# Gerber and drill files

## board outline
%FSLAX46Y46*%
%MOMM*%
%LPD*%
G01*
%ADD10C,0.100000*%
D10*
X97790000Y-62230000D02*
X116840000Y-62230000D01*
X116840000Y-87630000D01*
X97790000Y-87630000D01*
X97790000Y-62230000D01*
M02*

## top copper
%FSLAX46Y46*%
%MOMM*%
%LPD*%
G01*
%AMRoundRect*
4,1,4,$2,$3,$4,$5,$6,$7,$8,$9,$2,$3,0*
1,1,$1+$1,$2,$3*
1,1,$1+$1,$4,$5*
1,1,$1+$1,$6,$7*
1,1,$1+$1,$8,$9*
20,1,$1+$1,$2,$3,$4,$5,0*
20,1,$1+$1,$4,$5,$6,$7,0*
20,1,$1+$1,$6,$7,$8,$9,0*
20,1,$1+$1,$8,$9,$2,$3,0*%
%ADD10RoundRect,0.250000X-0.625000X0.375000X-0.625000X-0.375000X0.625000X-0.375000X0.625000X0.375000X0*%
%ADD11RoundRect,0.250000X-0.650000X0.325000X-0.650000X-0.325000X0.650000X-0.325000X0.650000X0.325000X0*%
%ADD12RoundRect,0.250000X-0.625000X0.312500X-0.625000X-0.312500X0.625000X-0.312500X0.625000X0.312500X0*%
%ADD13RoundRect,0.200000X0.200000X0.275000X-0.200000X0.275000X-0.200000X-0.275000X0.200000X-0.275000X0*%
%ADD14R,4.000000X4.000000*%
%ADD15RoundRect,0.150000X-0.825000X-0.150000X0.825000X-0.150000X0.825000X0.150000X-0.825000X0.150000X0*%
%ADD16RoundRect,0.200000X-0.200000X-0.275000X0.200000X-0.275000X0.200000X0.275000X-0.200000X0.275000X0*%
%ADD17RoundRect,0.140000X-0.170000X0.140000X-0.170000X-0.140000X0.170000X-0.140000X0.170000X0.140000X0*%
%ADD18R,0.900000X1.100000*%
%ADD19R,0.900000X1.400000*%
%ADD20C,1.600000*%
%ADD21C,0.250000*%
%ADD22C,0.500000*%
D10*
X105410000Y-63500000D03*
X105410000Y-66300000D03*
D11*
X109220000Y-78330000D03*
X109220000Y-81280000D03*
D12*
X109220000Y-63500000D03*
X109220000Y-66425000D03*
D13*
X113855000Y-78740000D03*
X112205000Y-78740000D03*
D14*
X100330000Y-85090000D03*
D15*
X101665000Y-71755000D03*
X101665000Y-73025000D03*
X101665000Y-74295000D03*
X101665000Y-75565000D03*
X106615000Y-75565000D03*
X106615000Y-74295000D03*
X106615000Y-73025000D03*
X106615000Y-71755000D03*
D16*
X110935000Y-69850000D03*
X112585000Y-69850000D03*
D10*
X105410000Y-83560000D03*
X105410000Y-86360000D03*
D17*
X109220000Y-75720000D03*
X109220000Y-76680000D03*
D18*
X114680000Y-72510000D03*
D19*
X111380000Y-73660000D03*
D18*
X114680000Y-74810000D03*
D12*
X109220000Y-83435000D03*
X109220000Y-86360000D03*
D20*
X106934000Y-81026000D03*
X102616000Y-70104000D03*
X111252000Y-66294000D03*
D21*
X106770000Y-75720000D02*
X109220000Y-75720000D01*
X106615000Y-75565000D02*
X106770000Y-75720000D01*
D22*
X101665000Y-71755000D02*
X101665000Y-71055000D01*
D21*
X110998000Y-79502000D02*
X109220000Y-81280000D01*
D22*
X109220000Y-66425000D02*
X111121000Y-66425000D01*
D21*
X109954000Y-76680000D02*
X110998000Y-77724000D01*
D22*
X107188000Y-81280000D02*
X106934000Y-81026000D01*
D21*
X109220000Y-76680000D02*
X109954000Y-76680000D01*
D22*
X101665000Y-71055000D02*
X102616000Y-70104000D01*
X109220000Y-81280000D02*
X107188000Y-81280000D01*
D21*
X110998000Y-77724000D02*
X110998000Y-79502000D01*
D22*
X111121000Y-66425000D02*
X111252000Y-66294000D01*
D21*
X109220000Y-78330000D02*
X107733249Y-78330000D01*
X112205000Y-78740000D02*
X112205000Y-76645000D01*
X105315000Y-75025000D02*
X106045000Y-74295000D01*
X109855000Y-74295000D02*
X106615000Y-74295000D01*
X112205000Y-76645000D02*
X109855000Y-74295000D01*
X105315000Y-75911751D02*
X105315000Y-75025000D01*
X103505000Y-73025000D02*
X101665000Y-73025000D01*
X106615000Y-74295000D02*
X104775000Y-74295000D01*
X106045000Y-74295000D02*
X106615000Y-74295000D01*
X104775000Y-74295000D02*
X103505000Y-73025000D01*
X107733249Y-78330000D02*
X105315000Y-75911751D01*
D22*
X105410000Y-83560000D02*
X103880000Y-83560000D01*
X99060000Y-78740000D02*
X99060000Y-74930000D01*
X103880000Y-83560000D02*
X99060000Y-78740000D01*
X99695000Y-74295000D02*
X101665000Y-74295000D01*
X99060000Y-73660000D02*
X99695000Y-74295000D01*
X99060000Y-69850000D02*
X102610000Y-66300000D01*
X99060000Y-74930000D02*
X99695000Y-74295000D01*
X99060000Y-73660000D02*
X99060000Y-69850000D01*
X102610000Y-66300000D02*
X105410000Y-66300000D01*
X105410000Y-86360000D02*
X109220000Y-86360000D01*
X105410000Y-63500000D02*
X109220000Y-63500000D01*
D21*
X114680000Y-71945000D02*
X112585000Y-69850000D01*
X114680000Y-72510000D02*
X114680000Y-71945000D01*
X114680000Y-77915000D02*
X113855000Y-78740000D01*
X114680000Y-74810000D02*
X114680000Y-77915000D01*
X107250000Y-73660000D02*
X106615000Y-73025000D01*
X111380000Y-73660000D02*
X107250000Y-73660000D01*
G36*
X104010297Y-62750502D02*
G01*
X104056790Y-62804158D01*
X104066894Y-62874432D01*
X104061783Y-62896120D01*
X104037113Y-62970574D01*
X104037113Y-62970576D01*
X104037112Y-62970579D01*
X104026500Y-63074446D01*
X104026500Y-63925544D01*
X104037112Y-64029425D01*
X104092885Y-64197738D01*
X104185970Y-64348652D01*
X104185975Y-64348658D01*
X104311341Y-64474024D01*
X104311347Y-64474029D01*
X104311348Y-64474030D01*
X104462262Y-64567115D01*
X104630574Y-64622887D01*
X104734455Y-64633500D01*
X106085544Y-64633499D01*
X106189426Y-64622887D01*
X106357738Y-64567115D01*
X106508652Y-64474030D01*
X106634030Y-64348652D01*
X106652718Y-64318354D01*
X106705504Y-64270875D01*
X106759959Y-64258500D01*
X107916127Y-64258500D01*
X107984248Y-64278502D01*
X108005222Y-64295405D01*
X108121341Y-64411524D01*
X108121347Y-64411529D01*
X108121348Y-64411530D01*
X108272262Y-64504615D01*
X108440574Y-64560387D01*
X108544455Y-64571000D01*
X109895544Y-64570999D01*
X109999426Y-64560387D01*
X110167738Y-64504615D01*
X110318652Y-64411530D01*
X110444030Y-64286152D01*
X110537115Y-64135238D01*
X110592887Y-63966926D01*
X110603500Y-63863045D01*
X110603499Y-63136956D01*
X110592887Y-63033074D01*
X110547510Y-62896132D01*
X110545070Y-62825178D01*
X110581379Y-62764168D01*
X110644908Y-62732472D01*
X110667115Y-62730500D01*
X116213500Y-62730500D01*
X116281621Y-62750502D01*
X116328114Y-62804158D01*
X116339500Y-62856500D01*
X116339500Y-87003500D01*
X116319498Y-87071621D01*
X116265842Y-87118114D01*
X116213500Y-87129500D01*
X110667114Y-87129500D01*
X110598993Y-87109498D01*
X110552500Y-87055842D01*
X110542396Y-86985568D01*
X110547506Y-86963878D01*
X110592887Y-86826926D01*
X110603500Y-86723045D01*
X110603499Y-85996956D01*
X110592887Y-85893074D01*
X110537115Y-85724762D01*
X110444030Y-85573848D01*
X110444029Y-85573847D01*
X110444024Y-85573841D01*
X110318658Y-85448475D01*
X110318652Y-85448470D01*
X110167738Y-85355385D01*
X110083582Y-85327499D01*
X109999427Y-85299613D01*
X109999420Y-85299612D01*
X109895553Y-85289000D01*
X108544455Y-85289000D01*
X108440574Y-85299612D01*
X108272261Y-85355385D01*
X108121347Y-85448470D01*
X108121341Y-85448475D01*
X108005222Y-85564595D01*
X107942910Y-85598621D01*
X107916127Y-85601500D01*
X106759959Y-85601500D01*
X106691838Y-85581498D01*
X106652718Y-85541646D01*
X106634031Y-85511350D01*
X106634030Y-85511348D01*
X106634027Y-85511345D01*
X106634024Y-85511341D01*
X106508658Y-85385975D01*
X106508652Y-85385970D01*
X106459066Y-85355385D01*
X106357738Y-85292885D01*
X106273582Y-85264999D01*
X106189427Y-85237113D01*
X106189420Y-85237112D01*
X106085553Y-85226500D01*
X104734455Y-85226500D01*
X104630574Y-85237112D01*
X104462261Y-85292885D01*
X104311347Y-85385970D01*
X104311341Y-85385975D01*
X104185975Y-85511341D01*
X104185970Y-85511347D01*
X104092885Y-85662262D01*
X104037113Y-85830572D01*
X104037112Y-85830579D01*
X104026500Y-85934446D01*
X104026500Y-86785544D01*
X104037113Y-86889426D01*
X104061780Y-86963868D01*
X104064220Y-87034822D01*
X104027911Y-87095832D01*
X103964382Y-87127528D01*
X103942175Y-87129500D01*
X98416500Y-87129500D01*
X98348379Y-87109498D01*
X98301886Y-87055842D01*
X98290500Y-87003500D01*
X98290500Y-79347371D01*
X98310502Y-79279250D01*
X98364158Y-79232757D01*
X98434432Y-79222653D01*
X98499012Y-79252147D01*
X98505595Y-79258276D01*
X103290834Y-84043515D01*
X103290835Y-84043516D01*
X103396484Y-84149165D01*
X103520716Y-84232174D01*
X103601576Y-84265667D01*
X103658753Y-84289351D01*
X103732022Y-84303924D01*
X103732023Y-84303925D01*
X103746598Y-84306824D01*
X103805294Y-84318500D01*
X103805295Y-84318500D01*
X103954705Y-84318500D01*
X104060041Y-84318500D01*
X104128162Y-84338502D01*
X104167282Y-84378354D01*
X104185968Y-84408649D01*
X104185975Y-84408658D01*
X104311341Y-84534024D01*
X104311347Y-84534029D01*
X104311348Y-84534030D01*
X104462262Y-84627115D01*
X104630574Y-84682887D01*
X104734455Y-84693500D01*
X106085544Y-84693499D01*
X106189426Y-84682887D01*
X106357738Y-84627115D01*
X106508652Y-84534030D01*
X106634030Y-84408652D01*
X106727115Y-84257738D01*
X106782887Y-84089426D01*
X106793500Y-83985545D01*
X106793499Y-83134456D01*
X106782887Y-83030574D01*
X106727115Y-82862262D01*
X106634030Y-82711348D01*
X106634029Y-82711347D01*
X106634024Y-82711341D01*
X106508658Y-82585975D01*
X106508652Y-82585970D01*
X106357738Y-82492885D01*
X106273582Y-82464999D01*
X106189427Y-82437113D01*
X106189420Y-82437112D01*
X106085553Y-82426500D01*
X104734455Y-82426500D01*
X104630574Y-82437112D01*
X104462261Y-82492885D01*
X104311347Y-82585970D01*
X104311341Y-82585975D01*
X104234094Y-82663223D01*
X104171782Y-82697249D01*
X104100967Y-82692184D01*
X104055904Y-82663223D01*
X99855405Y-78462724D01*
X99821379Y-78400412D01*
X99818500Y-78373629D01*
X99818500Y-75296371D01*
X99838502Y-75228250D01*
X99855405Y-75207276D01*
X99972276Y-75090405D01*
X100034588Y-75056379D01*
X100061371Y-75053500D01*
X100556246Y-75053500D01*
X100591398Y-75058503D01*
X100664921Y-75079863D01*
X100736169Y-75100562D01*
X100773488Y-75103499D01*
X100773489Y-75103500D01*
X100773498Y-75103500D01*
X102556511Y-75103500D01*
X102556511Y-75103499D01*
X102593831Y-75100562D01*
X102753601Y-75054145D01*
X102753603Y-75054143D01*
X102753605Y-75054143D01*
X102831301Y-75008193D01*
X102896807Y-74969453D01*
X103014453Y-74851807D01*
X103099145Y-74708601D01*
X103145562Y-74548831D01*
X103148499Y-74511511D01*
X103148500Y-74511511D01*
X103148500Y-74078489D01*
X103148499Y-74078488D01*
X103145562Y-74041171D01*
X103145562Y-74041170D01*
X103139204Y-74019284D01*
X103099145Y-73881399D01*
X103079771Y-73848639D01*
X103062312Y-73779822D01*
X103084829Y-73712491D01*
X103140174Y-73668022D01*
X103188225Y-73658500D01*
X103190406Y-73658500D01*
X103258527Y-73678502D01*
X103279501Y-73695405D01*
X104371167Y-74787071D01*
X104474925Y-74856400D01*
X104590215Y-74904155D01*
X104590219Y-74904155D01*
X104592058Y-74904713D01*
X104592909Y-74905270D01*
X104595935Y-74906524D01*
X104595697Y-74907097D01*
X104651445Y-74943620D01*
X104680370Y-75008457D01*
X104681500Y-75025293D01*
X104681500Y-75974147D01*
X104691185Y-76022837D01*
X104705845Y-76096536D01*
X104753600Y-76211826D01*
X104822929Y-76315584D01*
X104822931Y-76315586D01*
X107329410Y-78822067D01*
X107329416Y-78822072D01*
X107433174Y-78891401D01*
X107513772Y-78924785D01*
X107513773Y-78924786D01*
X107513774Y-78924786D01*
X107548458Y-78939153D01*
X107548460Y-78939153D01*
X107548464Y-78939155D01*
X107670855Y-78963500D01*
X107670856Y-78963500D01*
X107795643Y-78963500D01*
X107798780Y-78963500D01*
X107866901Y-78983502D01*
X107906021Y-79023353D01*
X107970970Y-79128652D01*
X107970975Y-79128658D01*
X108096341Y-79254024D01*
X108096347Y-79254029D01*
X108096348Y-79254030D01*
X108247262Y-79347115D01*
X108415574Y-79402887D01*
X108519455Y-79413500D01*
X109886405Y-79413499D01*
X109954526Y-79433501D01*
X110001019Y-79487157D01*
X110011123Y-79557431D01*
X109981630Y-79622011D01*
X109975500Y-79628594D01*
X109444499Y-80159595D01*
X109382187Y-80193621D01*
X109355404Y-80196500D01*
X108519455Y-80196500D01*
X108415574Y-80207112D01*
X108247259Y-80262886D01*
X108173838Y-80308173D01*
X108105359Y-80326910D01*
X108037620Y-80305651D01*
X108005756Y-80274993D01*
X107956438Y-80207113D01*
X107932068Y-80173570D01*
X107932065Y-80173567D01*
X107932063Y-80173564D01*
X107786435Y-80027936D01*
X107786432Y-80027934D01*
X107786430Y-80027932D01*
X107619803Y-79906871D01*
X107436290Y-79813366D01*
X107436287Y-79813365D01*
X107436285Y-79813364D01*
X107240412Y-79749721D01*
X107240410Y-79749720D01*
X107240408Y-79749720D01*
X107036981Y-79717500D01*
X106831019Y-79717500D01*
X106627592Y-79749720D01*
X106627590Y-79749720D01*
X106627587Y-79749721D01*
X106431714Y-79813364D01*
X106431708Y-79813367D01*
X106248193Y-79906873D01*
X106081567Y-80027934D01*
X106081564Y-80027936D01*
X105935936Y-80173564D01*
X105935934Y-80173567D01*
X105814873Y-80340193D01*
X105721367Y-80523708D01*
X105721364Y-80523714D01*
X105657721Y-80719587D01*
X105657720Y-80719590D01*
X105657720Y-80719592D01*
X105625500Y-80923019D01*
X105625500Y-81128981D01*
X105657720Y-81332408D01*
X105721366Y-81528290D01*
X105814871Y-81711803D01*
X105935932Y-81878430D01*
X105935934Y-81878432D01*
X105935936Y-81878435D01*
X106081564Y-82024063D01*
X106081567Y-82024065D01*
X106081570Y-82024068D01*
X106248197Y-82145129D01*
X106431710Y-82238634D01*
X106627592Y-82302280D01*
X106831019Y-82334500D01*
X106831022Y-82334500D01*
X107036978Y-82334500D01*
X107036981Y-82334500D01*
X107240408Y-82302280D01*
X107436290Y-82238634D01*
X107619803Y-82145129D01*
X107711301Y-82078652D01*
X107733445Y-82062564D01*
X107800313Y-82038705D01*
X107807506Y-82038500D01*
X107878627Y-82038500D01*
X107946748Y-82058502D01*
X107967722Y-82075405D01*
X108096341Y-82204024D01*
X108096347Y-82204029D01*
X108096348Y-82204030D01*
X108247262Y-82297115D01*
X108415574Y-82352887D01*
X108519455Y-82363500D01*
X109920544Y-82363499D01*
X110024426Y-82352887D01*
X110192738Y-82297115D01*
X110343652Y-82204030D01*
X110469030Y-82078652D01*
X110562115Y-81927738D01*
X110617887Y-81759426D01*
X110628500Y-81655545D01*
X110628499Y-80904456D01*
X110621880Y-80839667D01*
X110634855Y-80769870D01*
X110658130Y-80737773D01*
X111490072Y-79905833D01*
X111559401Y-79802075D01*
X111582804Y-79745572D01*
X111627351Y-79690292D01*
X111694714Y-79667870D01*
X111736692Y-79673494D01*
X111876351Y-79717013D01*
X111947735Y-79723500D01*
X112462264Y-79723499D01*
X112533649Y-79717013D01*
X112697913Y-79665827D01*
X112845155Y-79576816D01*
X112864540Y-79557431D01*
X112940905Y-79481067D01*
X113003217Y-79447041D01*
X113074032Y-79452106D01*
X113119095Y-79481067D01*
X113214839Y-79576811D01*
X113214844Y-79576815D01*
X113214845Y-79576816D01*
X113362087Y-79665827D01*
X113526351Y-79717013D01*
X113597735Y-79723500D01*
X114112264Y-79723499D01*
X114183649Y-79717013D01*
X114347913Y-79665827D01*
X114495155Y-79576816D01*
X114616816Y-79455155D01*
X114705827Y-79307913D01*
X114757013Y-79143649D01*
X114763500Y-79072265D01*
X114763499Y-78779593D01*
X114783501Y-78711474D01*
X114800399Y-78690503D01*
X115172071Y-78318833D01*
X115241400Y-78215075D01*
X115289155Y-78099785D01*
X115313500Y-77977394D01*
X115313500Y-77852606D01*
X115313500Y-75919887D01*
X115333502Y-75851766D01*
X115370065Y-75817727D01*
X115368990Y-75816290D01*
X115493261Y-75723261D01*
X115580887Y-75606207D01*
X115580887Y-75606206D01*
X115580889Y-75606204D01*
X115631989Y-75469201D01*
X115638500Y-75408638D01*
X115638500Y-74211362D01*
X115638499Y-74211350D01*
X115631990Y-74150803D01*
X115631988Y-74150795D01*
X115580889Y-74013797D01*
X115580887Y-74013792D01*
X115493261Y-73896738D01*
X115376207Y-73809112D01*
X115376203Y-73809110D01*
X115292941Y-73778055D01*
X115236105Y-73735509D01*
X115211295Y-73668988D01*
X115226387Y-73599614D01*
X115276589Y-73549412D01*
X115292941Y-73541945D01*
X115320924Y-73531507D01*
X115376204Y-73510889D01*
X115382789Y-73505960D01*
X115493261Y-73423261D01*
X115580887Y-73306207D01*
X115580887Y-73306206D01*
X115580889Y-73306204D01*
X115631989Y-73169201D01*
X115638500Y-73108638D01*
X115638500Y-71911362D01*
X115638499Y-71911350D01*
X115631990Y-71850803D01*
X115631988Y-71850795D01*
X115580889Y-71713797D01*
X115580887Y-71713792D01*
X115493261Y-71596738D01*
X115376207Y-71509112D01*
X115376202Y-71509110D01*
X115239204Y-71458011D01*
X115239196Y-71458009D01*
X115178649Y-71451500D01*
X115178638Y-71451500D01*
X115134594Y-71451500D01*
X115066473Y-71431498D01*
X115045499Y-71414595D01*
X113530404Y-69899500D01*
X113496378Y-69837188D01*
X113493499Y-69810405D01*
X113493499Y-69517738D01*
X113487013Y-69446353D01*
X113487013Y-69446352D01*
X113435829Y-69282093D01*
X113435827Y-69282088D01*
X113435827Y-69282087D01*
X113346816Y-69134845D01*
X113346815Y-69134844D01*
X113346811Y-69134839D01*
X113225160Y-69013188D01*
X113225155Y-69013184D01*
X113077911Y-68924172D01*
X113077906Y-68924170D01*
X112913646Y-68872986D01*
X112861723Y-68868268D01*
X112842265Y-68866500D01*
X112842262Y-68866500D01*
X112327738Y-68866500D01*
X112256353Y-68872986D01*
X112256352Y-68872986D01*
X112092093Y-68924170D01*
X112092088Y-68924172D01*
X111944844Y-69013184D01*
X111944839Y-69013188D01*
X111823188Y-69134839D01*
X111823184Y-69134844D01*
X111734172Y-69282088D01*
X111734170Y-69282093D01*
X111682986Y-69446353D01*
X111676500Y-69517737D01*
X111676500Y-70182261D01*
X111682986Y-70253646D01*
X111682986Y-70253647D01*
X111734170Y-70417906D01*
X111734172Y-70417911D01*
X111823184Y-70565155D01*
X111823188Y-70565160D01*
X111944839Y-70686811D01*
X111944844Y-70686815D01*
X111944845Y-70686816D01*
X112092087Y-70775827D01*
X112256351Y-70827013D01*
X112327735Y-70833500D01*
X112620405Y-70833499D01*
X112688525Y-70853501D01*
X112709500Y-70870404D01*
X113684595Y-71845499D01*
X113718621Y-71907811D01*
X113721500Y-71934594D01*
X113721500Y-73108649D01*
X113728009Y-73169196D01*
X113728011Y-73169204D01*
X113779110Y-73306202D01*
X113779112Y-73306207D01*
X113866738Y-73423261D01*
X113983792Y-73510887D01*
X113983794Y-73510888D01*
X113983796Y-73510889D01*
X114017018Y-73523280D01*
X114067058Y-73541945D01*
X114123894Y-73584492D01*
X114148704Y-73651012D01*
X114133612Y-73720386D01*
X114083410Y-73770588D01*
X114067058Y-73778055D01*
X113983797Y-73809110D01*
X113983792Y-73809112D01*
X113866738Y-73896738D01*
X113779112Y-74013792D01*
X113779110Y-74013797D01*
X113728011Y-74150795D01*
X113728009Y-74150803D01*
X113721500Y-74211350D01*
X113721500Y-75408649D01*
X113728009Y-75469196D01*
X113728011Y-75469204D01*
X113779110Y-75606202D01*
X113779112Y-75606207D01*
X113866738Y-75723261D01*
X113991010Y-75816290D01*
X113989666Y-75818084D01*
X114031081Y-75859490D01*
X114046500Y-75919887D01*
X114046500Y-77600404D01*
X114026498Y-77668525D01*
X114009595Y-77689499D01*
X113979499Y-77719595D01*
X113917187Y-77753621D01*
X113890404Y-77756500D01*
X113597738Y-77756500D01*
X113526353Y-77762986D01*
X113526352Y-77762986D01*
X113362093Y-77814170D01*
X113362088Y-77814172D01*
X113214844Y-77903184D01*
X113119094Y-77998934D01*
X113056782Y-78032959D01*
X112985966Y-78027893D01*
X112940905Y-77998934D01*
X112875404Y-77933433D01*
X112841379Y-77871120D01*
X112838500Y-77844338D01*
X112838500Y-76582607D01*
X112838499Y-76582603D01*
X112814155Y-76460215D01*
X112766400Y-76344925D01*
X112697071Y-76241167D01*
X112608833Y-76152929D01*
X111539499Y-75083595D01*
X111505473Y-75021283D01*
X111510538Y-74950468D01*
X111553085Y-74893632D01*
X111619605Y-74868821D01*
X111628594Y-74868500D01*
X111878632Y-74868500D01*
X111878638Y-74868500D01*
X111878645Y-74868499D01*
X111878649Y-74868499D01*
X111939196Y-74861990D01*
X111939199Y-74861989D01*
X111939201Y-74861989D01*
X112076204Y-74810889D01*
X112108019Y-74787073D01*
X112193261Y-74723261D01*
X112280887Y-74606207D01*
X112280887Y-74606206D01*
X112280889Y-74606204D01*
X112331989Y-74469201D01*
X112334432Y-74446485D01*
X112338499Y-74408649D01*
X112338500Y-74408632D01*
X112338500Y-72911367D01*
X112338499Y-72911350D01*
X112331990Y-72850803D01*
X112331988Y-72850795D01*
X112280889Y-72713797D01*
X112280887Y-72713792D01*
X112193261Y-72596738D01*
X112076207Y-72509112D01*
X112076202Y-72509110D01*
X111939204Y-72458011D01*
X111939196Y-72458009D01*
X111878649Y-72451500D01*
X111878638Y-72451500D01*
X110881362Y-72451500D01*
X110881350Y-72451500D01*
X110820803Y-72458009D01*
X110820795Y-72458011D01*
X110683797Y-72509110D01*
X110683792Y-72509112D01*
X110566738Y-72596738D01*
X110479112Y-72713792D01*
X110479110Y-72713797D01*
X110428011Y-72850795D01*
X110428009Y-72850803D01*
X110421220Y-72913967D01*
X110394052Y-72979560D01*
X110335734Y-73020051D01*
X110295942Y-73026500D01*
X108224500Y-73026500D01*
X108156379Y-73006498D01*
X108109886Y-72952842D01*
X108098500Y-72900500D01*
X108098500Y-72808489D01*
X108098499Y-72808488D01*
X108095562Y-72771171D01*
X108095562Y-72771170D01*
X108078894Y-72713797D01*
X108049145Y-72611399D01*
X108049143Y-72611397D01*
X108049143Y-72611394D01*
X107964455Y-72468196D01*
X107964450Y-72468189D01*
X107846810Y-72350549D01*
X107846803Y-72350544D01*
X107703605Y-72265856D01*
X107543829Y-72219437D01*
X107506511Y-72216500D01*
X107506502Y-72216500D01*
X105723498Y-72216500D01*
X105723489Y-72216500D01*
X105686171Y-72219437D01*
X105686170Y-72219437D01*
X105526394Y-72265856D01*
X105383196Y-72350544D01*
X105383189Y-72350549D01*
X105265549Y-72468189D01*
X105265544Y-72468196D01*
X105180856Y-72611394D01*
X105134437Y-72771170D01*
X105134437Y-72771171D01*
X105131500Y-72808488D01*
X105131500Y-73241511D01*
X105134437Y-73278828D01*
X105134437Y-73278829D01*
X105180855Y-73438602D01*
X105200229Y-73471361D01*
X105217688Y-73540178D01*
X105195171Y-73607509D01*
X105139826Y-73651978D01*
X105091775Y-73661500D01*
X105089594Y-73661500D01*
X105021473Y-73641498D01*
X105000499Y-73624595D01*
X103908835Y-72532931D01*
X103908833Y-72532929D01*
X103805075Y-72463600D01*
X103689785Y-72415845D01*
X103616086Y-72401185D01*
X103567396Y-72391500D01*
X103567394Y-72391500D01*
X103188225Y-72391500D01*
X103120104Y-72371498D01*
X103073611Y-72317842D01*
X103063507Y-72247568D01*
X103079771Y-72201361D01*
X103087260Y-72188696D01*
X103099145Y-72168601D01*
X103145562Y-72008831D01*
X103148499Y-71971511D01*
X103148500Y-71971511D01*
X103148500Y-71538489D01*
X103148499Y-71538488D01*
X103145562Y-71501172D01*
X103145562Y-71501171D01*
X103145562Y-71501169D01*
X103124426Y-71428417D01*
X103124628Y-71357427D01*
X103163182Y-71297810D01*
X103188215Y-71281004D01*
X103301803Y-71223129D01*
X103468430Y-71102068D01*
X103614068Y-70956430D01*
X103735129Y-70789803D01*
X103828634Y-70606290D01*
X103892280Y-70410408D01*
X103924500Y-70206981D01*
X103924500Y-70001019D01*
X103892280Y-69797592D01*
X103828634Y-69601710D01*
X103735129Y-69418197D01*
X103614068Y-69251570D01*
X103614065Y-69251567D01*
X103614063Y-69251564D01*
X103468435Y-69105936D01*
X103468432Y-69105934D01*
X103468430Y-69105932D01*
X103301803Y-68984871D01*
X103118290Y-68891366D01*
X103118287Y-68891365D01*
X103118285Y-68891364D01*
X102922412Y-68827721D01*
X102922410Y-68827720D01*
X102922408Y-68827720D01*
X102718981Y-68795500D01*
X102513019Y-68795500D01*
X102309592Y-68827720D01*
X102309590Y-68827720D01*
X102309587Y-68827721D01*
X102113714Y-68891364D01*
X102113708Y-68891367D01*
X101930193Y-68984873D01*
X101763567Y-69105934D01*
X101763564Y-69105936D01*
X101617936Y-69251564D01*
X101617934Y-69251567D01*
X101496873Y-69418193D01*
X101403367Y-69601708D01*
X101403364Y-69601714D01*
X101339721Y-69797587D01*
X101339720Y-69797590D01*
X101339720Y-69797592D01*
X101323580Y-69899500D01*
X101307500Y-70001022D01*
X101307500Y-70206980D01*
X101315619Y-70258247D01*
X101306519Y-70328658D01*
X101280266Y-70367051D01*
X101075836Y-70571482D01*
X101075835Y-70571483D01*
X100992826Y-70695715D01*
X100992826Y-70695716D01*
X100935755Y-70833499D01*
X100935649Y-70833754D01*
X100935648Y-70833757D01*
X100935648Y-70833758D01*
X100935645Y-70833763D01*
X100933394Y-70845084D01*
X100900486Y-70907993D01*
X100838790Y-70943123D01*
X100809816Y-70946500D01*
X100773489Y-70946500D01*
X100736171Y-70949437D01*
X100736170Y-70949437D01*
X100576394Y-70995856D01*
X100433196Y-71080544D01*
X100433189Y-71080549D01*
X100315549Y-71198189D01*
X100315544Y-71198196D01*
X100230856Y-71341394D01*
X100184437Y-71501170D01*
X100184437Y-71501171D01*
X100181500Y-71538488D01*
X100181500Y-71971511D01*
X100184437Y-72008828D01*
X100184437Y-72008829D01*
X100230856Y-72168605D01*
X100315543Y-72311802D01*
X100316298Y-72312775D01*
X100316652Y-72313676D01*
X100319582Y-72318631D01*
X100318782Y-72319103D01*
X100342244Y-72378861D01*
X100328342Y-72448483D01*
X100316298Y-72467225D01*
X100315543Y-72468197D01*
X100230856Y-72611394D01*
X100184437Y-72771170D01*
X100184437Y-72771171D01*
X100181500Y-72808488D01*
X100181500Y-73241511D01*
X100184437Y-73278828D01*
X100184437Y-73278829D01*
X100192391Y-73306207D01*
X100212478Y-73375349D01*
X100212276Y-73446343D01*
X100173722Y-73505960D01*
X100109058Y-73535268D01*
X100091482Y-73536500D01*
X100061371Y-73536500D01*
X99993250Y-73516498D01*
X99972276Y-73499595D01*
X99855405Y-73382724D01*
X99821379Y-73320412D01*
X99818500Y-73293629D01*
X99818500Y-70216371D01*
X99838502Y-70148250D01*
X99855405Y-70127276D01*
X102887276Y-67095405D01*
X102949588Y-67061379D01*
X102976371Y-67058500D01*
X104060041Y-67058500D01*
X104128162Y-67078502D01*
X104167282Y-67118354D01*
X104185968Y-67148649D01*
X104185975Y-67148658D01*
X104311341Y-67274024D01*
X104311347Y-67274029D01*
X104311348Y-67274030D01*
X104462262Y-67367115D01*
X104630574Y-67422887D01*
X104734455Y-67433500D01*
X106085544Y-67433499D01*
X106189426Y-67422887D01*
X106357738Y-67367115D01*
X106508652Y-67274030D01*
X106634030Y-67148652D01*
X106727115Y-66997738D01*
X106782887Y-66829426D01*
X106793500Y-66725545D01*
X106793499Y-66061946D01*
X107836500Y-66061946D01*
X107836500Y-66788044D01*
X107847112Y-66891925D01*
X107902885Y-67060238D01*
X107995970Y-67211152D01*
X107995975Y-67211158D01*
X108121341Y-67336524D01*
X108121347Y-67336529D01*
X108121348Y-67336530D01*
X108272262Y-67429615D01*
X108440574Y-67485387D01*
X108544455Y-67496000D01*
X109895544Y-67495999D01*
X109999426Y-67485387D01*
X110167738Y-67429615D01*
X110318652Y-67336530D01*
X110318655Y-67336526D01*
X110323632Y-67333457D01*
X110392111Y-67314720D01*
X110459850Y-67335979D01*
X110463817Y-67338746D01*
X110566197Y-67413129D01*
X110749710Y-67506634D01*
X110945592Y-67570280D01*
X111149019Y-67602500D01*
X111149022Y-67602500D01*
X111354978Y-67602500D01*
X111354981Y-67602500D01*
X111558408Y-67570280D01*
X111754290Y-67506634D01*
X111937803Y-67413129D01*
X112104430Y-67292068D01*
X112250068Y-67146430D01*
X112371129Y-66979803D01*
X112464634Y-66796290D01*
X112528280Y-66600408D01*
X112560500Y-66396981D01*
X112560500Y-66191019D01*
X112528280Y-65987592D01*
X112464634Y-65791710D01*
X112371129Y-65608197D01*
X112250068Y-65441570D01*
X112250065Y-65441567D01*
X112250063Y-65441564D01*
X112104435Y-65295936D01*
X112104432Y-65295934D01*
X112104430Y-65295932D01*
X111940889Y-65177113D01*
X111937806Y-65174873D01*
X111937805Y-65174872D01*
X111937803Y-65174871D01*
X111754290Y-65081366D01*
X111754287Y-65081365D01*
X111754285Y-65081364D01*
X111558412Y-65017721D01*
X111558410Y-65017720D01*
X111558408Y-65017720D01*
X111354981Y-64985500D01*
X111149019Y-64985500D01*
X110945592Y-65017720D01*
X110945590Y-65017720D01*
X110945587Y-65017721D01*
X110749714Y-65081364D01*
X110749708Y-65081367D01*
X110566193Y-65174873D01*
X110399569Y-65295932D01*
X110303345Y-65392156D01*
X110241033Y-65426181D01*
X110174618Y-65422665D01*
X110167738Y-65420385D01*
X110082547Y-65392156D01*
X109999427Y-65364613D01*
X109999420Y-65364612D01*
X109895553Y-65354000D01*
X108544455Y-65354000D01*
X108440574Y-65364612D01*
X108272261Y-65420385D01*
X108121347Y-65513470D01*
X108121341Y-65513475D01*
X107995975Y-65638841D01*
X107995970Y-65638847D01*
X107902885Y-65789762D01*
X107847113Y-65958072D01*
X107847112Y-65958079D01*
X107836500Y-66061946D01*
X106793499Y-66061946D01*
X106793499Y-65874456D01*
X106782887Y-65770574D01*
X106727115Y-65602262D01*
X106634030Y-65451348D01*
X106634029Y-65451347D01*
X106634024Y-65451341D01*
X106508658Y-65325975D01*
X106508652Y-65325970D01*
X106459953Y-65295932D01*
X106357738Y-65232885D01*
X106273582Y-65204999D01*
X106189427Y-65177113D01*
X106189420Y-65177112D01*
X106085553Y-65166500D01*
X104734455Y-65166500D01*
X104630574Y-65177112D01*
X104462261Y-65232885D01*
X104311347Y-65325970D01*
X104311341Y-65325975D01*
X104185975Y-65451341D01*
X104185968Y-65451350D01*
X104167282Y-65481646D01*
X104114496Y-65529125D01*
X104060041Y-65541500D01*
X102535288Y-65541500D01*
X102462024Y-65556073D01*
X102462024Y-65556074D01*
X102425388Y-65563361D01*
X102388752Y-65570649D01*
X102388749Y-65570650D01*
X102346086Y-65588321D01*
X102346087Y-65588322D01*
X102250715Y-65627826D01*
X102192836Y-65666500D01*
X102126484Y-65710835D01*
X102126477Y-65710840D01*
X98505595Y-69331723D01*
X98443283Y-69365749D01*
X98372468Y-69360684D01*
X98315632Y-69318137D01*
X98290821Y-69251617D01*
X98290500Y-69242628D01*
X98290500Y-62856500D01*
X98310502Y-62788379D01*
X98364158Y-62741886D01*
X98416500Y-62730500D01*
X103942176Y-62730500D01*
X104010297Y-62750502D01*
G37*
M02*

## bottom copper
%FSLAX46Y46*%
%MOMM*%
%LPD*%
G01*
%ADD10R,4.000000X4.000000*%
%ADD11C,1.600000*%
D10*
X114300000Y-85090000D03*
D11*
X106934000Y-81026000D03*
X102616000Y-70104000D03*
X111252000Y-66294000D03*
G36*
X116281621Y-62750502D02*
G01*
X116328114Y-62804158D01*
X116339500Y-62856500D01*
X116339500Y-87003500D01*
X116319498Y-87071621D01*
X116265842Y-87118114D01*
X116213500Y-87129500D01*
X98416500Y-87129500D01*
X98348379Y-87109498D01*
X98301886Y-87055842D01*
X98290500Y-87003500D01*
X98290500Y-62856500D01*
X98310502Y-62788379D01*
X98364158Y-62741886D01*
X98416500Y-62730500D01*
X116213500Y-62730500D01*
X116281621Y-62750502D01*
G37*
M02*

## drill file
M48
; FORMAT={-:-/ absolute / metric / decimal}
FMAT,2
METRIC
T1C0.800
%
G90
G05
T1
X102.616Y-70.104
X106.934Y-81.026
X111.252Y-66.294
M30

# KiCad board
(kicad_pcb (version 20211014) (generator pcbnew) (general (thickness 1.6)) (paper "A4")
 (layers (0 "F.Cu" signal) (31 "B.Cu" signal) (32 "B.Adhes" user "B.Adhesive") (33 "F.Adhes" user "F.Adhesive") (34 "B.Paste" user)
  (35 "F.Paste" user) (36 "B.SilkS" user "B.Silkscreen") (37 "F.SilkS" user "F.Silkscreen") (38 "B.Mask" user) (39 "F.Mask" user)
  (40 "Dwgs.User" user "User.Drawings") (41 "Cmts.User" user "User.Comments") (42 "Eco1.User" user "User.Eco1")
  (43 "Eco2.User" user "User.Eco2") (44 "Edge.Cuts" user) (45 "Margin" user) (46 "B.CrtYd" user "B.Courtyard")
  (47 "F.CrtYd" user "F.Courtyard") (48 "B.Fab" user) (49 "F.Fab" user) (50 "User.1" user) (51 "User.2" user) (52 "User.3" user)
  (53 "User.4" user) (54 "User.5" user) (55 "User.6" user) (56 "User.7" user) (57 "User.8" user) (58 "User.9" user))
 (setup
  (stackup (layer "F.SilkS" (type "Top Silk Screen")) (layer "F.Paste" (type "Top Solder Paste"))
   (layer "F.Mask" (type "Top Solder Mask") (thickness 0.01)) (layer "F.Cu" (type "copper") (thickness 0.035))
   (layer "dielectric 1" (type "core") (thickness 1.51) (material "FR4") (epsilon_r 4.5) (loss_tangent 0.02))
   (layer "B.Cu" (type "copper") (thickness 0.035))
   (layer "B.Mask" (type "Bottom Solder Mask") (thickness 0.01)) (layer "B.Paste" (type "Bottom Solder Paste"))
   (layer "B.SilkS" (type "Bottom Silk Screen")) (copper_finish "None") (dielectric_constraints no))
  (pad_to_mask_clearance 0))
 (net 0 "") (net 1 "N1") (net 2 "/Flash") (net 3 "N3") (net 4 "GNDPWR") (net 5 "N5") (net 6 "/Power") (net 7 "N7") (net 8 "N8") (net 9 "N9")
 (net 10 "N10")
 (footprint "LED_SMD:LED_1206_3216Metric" (layer "F.Cu") (at 105.41 64.9 -90)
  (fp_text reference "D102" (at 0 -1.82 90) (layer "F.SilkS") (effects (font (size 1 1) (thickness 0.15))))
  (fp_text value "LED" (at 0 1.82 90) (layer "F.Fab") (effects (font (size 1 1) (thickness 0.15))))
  (pad "1" smd roundrect (at -1.4 0 270) (size 1.25 1.75) (layers "F.Cu" "F.Paste" "F.Mask") (roundrect_rratio 0.2) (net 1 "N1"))
  (pad "2" smd roundrect (at 1.4 0 270) (size 1.25 1.75) (layers "F.Cu" "F.Paste" "F.Mask") (roundrect_rratio 0.2) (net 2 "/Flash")))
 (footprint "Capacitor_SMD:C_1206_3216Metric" (layer "F.Cu") (at 109.22 79.805 -90)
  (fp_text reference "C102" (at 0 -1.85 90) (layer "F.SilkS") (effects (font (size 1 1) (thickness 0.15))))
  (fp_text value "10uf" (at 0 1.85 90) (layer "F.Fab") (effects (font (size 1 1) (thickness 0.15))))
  (pad "1" smd roundrect (at -1.475 0 270) (size 1.15 1.8) (layers "F.Cu" "F.Paste" "F.Mask") (roundrect_rratio 0.217391) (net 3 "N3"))
  (pad "2" smd roundrect (at 1.475 0 270) (size 1.15 1.8) (layers "F.Cu" "F.Paste" "F.Mask") (roundrect_rratio 0.217391) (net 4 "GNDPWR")))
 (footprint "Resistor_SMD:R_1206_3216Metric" (layer "F.Cu") (at 109.22 64.9625 -90)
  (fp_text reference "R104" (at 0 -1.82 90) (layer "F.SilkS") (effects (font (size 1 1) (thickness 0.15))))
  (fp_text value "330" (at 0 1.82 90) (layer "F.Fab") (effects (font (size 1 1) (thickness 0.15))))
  (pad "1" smd roundrect (at -1.4625 0 270) (size 1.125 1.75) (layers "F.Cu" "F.Paste" "F.Mask") (roundrect_rratio 0.222222) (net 1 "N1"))
  (pad "2" smd roundrect (at 1.4625 0 270) (size 1.125 1.75) (layers "F.Cu" "F.Paste" "F.Mask") (roundrect_rratio 0.222222) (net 4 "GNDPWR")))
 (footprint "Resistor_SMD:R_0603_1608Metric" (layer "F.Cu") (at 113.03 78.74 180)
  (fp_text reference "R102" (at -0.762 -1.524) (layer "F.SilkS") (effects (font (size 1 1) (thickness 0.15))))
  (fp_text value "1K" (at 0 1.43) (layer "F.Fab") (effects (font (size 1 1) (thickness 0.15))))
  (pad "1" smd roundrect (at -0.825 0 180) (size 0.8 0.95) (layers "F.Cu" "F.Paste" "F.Mask") (roundrect_rratio 0.25) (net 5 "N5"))
  (pad "2" smd roundrect (at 0.825 0 180) (size 0.8 0.95) (layers "F.Cu" "F.Paste" "F.Mask") (roundrect_rratio 0.25) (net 3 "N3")))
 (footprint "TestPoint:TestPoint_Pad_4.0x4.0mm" (layer "F.Cu") (at 100.33 85.09)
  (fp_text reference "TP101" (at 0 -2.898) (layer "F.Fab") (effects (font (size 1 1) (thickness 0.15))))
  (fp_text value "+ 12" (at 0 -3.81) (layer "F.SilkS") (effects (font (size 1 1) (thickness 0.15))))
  (pad "1" smd rect (at 0 0) (size 4 4) (layers "F.Cu" "F.Mask") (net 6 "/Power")))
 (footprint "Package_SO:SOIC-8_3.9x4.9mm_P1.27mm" (layer "F.Cu") (at 104.14 73.66)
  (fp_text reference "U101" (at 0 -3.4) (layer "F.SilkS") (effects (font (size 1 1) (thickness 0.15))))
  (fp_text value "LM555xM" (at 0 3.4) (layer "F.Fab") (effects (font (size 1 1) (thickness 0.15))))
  (pad "1" smd roundrect (at -2.475 -1.905) (size 1.95 0.6) (layers "F.Cu" "F.Paste" "F.Mask") (roundrect_rratio 0.25) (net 4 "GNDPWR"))
  (pad "2" smd roundrect (at -2.475 -0.635) (size 1.95 0.6) (layers "F.Cu" "F.Paste" "F.Mask") (roundrect_rratio 0.25) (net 3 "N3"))
  (pad "3" smd roundrect (at -2.475 0.635) (size 1.95 0.6) (layers "F.Cu" "F.Paste" "F.Mask") (roundrect_rratio 0.25) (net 2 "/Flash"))
  (pad "4" smd roundrect (at -2.475 1.905) (size 1.95 0.6) (layers "F.Cu" "F.Paste" "F.Mask") (roundrect_rratio 0.25) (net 6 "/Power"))
  (pad "5" smd roundrect (at 2.475 1.905) (size 1.95 0.6) (layers "F.Cu" "F.Paste" "F.Mask") (roundrect_rratio 0.25) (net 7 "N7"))
  (pad "6" smd roundrect (at 2.475 0.635) (size 1.95 0.6) (layers "F.Cu" "F.Paste" "F.Mask") (roundrect_rratio 0.25) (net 3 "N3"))
  (pad "7" smd roundrect (at 2.475 -0.635) (size 1.95 0.6) (layers "F.Cu" "F.Paste" "F.Mask") (roundrect_rratio 0.25) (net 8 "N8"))
  (pad "8" smd roundrect (at 2.475 -1.905) (size 1.95 0.6) (layers "F.Cu" "F.Paste" "F.Mask") (roundrect_rratio 0.25) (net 6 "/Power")))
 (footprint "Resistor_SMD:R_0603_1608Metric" (layer "F.Cu") (at 111.76 69.85)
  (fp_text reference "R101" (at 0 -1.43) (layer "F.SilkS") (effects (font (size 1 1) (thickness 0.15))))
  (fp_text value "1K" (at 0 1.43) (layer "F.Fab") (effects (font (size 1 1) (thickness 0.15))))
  (pad "1" smd roundrect (at -0.825 0) (size 0.8 0.95) (layers "F.Cu" "F.Paste" "F.Mask") (roundrect_rratio 0.25) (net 6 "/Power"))
  (pad "2" smd roundrect (at 0.825 0) (size 0.8 0.95) (layers "F.Cu" "F.Paste" "F.Mask") (roundrect_rratio 0.25) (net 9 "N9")))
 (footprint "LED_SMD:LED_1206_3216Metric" (layer "F.Cu") (at 105.41 84.96 -90)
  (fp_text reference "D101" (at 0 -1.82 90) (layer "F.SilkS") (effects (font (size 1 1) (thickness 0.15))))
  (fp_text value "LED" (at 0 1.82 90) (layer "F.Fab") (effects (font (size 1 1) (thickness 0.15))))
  (pad "1" smd roundrect (at -1.4 0 270) (size 1.25 1.75) (layers "F.Cu" "F.Paste" "F.Mask") (roundrect_rratio 0.2) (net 2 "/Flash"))
  (pad "2" smd roundrect (at 1.4 0 270) (size 1.25 1.75) (layers "F.Cu" "F.Paste" "F.Mask") (roundrect_rratio 0.2) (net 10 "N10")))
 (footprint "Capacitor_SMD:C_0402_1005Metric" (layer "F.Cu") (at 109.22 76.2 -90)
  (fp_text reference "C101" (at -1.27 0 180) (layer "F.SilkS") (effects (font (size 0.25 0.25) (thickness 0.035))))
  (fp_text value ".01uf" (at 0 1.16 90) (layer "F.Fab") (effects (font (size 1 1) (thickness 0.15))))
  (pad "1" smd roundrect (at -0.48 0 270) (size 0.56 0.62) (layers "F.Cu" "F.Paste" "F.Mask") (roundrect_rratio 0.25) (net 7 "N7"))
  (pad "2" smd roundrect (at 0.48 0 270) (size 0.56 0.62) (layers "F.Cu" "F.Paste" "F.Mask") (roundrect_rratio 0.25) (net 4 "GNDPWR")))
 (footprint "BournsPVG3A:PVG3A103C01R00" (layer "F.Cu") (at 113.03 73.66 90)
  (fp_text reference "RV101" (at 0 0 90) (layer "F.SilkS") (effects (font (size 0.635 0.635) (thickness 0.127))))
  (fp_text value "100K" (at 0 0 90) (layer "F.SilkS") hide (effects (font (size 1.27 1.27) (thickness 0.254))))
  (pad "1" smd rect locked (at 1.15 1.65 180) (size 0.9 1.1) (layers "F.Cu" "F.Paste" "F.Mask") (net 9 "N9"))
  (pad "2" smd rect locked (at 0 -1.65 180) (size 0.9 1.4) (layers "F.Cu" "F.Paste" "F.Mask") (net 8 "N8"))
  (pad "3" smd rect locked (at -1.15 1.65 180) (size 0.9 1.1) (layers "F.Cu" "F.Paste" "F.Mask") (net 5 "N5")))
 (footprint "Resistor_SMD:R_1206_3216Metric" (layer "F.Cu") (at 109.22 84.8975 -90)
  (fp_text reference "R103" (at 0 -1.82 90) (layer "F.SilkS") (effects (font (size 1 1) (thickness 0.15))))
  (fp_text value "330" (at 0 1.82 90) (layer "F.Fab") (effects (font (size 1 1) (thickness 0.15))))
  (pad "1" smd roundrect (at -1.4625 0 270) (size 1.125 1.75) (layers "F.Cu" "F.Paste" "F.Mask") (roundrect_rratio 0.222222)
   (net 6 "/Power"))
  (pad "2" smd roundrect (at 1.4625 0 270) (size 1.125 1.75) (layers "F.Cu" "F.Paste" "F.Mask") (roundrect_rratio 0.222222) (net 10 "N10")))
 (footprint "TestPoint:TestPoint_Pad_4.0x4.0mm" (layer "B.Cu") (at 114.3 85.09 180)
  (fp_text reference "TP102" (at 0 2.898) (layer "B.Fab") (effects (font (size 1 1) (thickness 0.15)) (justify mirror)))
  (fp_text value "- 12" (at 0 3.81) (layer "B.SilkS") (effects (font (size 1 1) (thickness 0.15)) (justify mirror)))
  (pad "1" smd rect (at 0 0 180) (size 4 4) (layers "B.Cu" "B.Mask") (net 4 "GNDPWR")))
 (gr_rect (start 97.79 62.23) (end 116.84 87.63) (layer "Edge.Cuts") (width 0.1) (fill none))
 (segment (start 106.77 75.72) (end 109.22 75.72) (width 0.25) (layer "F.Cu") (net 7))
 (segment (start 106.615 75.565) (end 106.77 75.72) (width 0.25) (layer "F.Cu") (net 7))
 (segment (start 101.665 71.755) (end 101.665 71.055) (width 0.5) (layer "F.Cu") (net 4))
 (segment (start 110.998 79.502) (end 109.22 81.28) (width 0.25) (layer "F.Cu") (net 4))
 (segment (start 109.22 66.425) (end 111.121 66.425) (width 0.5) (layer "F.Cu") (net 4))
 (segment (start 109.954 76.68) (end 110.998 77.724) (width 0.25) (layer "F.Cu") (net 4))
 (segment (start 107.188 81.28) (end 106.934 81.026) (width 0.5) (layer "F.Cu") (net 4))
 (segment (start 109.22 76.68) (end 109.954 76.68) (width 0.25) (layer "F.Cu") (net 4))
 (segment (start 101.665 71.055) (end 102.616 70.104) (width 0.5) (layer "F.Cu") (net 4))
 (segment (start 109.22 81.28) (end 107.188 81.28) (width 0.5) (layer "F.Cu") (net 4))
 (segment (start 110.998 77.724) (end 110.998 79.502) (width 0.25) (layer "F.Cu") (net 4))
 (segment (start 111.121 66.425) (end 111.252 66.294) (width 0.5) (layer "F.Cu") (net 4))
 (via (at 106.934 81.026) (size 1.6) (drill 0.8) (layers "F.Cu" "B.Cu") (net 4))
 (via (at 102.616 70.104) (size 1.6) (drill 0.8) (layers "F.Cu" "B.Cu") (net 4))
 (via (at 111.252 66.294) (size 1.6) (drill 0.8) (layers "F.Cu" "B.Cu") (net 4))
 (segment (start 109.22 78.33) (end 107.733249 78.33) (width 0.25) (layer "F.Cu") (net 3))
 (segment (start 112.205 78.74) (end 112.205 76.645) (width 0.25) (layer "F.Cu") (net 3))
 (segment (start 105.315 75.025) (end 106.045 74.295) (width 0.25) (layer "F.Cu") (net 3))
 (segment (start 109.855 74.295) (end 106.615 74.295) (width 0.25) (layer "F.Cu") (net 3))
 (segment (start 112.205 76.645) (end 109.855 74.295) (width 0.25) (layer "F.Cu") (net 3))
 (segment (start 105.315 75.911751) (end 105.315 75.025) (width 0.25) (layer "F.Cu") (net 3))
 (segment (start 103.505 73.025) (end 101.665 73.025) (width 0.25) (layer "F.Cu") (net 3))
 (segment (start 106.615 74.295) (end 104.775 74.295) (width 0.25) (layer "F.Cu") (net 3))
 (segment (start 106.045 74.295) (end 106.615 74.295) (width 0.25) (layer "F.Cu") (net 3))
 (segment (start 104.775 74.295) (end 103.505 73.025) (width 0.25) (layer "F.Cu") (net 3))
 (segment (start 107.733249 78.33) (end 105.315 75.911751) (width 0.25) (layer "F.Cu") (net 3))
 (segment (start 105.41 83.56) (end 103.88 83.56) (width 0.5) (layer "F.Cu") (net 2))
 (segment (start 99.06 78.74) (end 99.06 74.93) (width 0.5) (layer "F.Cu") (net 2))
 (segment (start 103.88 83.56) (end 99.06 78.74) (width 0.5) (layer "F.Cu") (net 2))
 (segment (start 99.695 74.295) (end 101.665 74.295) (width 0.5) (layer "F.Cu") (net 2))
 (segment (start 99.06 73.66) (end 99.695 74.295) (width 0.5) (layer "F.Cu") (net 2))
 (segment (start 99.06 69.85) (end 102.61 66.3) (width 0.5) (layer "F.Cu") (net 2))
 (segment (start 99.06 74.93) (end 99.695 74.295) (width 0.5) (layer "F.Cu") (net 2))
 (segment (start 99.06 73.66) (end 99.06 69.85) (width 0.5) (layer "F.Cu") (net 2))
 (segment (start 102.61 66.3) (end 105.41 66.3) (width 0.5) (layer "F.Cu") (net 2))
 (segment (start 105.41 86.36) (end 109.22 86.36) (width 0.5) (layer "F.Cu") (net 10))
 (segment (start 105.41 63.5) (end 109.22 63.5) (width 0.5) (layer "F.Cu") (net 1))
 (segment (start 114.68 71.945) (end 112.585 69.85) (width 0.25) (layer "F.Cu") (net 9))
 (segment (start 114.68 72.51) (end 114.68 71.945) (width 0.25) (layer "F.Cu") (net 9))
 (segment (start 114.68 77.915) (end 113.855 78.74) (width 0.25) (layer "F.Cu") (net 5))
 (segment (start 114.68 74.81) (end 114.68 77.915) (width 0.25) (layer "F.Cu") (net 5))
 (segment (start 107.25 73.66) (end 106.615 73.025) (width 0.25) (layer "F.Cu") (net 8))
 (segment (start 111.38 73.66) (end 107.25 73.66) (width 0.25) (layer "F.Cu") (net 8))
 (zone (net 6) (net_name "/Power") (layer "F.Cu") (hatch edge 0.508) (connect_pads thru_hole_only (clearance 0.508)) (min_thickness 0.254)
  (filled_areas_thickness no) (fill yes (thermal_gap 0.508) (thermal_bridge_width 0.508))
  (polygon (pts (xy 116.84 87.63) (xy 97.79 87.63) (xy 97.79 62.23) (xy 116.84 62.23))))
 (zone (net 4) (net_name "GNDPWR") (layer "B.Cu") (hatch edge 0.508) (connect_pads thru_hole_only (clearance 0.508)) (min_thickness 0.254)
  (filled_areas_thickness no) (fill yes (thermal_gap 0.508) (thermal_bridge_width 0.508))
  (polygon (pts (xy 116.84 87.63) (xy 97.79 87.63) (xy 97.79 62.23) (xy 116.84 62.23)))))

